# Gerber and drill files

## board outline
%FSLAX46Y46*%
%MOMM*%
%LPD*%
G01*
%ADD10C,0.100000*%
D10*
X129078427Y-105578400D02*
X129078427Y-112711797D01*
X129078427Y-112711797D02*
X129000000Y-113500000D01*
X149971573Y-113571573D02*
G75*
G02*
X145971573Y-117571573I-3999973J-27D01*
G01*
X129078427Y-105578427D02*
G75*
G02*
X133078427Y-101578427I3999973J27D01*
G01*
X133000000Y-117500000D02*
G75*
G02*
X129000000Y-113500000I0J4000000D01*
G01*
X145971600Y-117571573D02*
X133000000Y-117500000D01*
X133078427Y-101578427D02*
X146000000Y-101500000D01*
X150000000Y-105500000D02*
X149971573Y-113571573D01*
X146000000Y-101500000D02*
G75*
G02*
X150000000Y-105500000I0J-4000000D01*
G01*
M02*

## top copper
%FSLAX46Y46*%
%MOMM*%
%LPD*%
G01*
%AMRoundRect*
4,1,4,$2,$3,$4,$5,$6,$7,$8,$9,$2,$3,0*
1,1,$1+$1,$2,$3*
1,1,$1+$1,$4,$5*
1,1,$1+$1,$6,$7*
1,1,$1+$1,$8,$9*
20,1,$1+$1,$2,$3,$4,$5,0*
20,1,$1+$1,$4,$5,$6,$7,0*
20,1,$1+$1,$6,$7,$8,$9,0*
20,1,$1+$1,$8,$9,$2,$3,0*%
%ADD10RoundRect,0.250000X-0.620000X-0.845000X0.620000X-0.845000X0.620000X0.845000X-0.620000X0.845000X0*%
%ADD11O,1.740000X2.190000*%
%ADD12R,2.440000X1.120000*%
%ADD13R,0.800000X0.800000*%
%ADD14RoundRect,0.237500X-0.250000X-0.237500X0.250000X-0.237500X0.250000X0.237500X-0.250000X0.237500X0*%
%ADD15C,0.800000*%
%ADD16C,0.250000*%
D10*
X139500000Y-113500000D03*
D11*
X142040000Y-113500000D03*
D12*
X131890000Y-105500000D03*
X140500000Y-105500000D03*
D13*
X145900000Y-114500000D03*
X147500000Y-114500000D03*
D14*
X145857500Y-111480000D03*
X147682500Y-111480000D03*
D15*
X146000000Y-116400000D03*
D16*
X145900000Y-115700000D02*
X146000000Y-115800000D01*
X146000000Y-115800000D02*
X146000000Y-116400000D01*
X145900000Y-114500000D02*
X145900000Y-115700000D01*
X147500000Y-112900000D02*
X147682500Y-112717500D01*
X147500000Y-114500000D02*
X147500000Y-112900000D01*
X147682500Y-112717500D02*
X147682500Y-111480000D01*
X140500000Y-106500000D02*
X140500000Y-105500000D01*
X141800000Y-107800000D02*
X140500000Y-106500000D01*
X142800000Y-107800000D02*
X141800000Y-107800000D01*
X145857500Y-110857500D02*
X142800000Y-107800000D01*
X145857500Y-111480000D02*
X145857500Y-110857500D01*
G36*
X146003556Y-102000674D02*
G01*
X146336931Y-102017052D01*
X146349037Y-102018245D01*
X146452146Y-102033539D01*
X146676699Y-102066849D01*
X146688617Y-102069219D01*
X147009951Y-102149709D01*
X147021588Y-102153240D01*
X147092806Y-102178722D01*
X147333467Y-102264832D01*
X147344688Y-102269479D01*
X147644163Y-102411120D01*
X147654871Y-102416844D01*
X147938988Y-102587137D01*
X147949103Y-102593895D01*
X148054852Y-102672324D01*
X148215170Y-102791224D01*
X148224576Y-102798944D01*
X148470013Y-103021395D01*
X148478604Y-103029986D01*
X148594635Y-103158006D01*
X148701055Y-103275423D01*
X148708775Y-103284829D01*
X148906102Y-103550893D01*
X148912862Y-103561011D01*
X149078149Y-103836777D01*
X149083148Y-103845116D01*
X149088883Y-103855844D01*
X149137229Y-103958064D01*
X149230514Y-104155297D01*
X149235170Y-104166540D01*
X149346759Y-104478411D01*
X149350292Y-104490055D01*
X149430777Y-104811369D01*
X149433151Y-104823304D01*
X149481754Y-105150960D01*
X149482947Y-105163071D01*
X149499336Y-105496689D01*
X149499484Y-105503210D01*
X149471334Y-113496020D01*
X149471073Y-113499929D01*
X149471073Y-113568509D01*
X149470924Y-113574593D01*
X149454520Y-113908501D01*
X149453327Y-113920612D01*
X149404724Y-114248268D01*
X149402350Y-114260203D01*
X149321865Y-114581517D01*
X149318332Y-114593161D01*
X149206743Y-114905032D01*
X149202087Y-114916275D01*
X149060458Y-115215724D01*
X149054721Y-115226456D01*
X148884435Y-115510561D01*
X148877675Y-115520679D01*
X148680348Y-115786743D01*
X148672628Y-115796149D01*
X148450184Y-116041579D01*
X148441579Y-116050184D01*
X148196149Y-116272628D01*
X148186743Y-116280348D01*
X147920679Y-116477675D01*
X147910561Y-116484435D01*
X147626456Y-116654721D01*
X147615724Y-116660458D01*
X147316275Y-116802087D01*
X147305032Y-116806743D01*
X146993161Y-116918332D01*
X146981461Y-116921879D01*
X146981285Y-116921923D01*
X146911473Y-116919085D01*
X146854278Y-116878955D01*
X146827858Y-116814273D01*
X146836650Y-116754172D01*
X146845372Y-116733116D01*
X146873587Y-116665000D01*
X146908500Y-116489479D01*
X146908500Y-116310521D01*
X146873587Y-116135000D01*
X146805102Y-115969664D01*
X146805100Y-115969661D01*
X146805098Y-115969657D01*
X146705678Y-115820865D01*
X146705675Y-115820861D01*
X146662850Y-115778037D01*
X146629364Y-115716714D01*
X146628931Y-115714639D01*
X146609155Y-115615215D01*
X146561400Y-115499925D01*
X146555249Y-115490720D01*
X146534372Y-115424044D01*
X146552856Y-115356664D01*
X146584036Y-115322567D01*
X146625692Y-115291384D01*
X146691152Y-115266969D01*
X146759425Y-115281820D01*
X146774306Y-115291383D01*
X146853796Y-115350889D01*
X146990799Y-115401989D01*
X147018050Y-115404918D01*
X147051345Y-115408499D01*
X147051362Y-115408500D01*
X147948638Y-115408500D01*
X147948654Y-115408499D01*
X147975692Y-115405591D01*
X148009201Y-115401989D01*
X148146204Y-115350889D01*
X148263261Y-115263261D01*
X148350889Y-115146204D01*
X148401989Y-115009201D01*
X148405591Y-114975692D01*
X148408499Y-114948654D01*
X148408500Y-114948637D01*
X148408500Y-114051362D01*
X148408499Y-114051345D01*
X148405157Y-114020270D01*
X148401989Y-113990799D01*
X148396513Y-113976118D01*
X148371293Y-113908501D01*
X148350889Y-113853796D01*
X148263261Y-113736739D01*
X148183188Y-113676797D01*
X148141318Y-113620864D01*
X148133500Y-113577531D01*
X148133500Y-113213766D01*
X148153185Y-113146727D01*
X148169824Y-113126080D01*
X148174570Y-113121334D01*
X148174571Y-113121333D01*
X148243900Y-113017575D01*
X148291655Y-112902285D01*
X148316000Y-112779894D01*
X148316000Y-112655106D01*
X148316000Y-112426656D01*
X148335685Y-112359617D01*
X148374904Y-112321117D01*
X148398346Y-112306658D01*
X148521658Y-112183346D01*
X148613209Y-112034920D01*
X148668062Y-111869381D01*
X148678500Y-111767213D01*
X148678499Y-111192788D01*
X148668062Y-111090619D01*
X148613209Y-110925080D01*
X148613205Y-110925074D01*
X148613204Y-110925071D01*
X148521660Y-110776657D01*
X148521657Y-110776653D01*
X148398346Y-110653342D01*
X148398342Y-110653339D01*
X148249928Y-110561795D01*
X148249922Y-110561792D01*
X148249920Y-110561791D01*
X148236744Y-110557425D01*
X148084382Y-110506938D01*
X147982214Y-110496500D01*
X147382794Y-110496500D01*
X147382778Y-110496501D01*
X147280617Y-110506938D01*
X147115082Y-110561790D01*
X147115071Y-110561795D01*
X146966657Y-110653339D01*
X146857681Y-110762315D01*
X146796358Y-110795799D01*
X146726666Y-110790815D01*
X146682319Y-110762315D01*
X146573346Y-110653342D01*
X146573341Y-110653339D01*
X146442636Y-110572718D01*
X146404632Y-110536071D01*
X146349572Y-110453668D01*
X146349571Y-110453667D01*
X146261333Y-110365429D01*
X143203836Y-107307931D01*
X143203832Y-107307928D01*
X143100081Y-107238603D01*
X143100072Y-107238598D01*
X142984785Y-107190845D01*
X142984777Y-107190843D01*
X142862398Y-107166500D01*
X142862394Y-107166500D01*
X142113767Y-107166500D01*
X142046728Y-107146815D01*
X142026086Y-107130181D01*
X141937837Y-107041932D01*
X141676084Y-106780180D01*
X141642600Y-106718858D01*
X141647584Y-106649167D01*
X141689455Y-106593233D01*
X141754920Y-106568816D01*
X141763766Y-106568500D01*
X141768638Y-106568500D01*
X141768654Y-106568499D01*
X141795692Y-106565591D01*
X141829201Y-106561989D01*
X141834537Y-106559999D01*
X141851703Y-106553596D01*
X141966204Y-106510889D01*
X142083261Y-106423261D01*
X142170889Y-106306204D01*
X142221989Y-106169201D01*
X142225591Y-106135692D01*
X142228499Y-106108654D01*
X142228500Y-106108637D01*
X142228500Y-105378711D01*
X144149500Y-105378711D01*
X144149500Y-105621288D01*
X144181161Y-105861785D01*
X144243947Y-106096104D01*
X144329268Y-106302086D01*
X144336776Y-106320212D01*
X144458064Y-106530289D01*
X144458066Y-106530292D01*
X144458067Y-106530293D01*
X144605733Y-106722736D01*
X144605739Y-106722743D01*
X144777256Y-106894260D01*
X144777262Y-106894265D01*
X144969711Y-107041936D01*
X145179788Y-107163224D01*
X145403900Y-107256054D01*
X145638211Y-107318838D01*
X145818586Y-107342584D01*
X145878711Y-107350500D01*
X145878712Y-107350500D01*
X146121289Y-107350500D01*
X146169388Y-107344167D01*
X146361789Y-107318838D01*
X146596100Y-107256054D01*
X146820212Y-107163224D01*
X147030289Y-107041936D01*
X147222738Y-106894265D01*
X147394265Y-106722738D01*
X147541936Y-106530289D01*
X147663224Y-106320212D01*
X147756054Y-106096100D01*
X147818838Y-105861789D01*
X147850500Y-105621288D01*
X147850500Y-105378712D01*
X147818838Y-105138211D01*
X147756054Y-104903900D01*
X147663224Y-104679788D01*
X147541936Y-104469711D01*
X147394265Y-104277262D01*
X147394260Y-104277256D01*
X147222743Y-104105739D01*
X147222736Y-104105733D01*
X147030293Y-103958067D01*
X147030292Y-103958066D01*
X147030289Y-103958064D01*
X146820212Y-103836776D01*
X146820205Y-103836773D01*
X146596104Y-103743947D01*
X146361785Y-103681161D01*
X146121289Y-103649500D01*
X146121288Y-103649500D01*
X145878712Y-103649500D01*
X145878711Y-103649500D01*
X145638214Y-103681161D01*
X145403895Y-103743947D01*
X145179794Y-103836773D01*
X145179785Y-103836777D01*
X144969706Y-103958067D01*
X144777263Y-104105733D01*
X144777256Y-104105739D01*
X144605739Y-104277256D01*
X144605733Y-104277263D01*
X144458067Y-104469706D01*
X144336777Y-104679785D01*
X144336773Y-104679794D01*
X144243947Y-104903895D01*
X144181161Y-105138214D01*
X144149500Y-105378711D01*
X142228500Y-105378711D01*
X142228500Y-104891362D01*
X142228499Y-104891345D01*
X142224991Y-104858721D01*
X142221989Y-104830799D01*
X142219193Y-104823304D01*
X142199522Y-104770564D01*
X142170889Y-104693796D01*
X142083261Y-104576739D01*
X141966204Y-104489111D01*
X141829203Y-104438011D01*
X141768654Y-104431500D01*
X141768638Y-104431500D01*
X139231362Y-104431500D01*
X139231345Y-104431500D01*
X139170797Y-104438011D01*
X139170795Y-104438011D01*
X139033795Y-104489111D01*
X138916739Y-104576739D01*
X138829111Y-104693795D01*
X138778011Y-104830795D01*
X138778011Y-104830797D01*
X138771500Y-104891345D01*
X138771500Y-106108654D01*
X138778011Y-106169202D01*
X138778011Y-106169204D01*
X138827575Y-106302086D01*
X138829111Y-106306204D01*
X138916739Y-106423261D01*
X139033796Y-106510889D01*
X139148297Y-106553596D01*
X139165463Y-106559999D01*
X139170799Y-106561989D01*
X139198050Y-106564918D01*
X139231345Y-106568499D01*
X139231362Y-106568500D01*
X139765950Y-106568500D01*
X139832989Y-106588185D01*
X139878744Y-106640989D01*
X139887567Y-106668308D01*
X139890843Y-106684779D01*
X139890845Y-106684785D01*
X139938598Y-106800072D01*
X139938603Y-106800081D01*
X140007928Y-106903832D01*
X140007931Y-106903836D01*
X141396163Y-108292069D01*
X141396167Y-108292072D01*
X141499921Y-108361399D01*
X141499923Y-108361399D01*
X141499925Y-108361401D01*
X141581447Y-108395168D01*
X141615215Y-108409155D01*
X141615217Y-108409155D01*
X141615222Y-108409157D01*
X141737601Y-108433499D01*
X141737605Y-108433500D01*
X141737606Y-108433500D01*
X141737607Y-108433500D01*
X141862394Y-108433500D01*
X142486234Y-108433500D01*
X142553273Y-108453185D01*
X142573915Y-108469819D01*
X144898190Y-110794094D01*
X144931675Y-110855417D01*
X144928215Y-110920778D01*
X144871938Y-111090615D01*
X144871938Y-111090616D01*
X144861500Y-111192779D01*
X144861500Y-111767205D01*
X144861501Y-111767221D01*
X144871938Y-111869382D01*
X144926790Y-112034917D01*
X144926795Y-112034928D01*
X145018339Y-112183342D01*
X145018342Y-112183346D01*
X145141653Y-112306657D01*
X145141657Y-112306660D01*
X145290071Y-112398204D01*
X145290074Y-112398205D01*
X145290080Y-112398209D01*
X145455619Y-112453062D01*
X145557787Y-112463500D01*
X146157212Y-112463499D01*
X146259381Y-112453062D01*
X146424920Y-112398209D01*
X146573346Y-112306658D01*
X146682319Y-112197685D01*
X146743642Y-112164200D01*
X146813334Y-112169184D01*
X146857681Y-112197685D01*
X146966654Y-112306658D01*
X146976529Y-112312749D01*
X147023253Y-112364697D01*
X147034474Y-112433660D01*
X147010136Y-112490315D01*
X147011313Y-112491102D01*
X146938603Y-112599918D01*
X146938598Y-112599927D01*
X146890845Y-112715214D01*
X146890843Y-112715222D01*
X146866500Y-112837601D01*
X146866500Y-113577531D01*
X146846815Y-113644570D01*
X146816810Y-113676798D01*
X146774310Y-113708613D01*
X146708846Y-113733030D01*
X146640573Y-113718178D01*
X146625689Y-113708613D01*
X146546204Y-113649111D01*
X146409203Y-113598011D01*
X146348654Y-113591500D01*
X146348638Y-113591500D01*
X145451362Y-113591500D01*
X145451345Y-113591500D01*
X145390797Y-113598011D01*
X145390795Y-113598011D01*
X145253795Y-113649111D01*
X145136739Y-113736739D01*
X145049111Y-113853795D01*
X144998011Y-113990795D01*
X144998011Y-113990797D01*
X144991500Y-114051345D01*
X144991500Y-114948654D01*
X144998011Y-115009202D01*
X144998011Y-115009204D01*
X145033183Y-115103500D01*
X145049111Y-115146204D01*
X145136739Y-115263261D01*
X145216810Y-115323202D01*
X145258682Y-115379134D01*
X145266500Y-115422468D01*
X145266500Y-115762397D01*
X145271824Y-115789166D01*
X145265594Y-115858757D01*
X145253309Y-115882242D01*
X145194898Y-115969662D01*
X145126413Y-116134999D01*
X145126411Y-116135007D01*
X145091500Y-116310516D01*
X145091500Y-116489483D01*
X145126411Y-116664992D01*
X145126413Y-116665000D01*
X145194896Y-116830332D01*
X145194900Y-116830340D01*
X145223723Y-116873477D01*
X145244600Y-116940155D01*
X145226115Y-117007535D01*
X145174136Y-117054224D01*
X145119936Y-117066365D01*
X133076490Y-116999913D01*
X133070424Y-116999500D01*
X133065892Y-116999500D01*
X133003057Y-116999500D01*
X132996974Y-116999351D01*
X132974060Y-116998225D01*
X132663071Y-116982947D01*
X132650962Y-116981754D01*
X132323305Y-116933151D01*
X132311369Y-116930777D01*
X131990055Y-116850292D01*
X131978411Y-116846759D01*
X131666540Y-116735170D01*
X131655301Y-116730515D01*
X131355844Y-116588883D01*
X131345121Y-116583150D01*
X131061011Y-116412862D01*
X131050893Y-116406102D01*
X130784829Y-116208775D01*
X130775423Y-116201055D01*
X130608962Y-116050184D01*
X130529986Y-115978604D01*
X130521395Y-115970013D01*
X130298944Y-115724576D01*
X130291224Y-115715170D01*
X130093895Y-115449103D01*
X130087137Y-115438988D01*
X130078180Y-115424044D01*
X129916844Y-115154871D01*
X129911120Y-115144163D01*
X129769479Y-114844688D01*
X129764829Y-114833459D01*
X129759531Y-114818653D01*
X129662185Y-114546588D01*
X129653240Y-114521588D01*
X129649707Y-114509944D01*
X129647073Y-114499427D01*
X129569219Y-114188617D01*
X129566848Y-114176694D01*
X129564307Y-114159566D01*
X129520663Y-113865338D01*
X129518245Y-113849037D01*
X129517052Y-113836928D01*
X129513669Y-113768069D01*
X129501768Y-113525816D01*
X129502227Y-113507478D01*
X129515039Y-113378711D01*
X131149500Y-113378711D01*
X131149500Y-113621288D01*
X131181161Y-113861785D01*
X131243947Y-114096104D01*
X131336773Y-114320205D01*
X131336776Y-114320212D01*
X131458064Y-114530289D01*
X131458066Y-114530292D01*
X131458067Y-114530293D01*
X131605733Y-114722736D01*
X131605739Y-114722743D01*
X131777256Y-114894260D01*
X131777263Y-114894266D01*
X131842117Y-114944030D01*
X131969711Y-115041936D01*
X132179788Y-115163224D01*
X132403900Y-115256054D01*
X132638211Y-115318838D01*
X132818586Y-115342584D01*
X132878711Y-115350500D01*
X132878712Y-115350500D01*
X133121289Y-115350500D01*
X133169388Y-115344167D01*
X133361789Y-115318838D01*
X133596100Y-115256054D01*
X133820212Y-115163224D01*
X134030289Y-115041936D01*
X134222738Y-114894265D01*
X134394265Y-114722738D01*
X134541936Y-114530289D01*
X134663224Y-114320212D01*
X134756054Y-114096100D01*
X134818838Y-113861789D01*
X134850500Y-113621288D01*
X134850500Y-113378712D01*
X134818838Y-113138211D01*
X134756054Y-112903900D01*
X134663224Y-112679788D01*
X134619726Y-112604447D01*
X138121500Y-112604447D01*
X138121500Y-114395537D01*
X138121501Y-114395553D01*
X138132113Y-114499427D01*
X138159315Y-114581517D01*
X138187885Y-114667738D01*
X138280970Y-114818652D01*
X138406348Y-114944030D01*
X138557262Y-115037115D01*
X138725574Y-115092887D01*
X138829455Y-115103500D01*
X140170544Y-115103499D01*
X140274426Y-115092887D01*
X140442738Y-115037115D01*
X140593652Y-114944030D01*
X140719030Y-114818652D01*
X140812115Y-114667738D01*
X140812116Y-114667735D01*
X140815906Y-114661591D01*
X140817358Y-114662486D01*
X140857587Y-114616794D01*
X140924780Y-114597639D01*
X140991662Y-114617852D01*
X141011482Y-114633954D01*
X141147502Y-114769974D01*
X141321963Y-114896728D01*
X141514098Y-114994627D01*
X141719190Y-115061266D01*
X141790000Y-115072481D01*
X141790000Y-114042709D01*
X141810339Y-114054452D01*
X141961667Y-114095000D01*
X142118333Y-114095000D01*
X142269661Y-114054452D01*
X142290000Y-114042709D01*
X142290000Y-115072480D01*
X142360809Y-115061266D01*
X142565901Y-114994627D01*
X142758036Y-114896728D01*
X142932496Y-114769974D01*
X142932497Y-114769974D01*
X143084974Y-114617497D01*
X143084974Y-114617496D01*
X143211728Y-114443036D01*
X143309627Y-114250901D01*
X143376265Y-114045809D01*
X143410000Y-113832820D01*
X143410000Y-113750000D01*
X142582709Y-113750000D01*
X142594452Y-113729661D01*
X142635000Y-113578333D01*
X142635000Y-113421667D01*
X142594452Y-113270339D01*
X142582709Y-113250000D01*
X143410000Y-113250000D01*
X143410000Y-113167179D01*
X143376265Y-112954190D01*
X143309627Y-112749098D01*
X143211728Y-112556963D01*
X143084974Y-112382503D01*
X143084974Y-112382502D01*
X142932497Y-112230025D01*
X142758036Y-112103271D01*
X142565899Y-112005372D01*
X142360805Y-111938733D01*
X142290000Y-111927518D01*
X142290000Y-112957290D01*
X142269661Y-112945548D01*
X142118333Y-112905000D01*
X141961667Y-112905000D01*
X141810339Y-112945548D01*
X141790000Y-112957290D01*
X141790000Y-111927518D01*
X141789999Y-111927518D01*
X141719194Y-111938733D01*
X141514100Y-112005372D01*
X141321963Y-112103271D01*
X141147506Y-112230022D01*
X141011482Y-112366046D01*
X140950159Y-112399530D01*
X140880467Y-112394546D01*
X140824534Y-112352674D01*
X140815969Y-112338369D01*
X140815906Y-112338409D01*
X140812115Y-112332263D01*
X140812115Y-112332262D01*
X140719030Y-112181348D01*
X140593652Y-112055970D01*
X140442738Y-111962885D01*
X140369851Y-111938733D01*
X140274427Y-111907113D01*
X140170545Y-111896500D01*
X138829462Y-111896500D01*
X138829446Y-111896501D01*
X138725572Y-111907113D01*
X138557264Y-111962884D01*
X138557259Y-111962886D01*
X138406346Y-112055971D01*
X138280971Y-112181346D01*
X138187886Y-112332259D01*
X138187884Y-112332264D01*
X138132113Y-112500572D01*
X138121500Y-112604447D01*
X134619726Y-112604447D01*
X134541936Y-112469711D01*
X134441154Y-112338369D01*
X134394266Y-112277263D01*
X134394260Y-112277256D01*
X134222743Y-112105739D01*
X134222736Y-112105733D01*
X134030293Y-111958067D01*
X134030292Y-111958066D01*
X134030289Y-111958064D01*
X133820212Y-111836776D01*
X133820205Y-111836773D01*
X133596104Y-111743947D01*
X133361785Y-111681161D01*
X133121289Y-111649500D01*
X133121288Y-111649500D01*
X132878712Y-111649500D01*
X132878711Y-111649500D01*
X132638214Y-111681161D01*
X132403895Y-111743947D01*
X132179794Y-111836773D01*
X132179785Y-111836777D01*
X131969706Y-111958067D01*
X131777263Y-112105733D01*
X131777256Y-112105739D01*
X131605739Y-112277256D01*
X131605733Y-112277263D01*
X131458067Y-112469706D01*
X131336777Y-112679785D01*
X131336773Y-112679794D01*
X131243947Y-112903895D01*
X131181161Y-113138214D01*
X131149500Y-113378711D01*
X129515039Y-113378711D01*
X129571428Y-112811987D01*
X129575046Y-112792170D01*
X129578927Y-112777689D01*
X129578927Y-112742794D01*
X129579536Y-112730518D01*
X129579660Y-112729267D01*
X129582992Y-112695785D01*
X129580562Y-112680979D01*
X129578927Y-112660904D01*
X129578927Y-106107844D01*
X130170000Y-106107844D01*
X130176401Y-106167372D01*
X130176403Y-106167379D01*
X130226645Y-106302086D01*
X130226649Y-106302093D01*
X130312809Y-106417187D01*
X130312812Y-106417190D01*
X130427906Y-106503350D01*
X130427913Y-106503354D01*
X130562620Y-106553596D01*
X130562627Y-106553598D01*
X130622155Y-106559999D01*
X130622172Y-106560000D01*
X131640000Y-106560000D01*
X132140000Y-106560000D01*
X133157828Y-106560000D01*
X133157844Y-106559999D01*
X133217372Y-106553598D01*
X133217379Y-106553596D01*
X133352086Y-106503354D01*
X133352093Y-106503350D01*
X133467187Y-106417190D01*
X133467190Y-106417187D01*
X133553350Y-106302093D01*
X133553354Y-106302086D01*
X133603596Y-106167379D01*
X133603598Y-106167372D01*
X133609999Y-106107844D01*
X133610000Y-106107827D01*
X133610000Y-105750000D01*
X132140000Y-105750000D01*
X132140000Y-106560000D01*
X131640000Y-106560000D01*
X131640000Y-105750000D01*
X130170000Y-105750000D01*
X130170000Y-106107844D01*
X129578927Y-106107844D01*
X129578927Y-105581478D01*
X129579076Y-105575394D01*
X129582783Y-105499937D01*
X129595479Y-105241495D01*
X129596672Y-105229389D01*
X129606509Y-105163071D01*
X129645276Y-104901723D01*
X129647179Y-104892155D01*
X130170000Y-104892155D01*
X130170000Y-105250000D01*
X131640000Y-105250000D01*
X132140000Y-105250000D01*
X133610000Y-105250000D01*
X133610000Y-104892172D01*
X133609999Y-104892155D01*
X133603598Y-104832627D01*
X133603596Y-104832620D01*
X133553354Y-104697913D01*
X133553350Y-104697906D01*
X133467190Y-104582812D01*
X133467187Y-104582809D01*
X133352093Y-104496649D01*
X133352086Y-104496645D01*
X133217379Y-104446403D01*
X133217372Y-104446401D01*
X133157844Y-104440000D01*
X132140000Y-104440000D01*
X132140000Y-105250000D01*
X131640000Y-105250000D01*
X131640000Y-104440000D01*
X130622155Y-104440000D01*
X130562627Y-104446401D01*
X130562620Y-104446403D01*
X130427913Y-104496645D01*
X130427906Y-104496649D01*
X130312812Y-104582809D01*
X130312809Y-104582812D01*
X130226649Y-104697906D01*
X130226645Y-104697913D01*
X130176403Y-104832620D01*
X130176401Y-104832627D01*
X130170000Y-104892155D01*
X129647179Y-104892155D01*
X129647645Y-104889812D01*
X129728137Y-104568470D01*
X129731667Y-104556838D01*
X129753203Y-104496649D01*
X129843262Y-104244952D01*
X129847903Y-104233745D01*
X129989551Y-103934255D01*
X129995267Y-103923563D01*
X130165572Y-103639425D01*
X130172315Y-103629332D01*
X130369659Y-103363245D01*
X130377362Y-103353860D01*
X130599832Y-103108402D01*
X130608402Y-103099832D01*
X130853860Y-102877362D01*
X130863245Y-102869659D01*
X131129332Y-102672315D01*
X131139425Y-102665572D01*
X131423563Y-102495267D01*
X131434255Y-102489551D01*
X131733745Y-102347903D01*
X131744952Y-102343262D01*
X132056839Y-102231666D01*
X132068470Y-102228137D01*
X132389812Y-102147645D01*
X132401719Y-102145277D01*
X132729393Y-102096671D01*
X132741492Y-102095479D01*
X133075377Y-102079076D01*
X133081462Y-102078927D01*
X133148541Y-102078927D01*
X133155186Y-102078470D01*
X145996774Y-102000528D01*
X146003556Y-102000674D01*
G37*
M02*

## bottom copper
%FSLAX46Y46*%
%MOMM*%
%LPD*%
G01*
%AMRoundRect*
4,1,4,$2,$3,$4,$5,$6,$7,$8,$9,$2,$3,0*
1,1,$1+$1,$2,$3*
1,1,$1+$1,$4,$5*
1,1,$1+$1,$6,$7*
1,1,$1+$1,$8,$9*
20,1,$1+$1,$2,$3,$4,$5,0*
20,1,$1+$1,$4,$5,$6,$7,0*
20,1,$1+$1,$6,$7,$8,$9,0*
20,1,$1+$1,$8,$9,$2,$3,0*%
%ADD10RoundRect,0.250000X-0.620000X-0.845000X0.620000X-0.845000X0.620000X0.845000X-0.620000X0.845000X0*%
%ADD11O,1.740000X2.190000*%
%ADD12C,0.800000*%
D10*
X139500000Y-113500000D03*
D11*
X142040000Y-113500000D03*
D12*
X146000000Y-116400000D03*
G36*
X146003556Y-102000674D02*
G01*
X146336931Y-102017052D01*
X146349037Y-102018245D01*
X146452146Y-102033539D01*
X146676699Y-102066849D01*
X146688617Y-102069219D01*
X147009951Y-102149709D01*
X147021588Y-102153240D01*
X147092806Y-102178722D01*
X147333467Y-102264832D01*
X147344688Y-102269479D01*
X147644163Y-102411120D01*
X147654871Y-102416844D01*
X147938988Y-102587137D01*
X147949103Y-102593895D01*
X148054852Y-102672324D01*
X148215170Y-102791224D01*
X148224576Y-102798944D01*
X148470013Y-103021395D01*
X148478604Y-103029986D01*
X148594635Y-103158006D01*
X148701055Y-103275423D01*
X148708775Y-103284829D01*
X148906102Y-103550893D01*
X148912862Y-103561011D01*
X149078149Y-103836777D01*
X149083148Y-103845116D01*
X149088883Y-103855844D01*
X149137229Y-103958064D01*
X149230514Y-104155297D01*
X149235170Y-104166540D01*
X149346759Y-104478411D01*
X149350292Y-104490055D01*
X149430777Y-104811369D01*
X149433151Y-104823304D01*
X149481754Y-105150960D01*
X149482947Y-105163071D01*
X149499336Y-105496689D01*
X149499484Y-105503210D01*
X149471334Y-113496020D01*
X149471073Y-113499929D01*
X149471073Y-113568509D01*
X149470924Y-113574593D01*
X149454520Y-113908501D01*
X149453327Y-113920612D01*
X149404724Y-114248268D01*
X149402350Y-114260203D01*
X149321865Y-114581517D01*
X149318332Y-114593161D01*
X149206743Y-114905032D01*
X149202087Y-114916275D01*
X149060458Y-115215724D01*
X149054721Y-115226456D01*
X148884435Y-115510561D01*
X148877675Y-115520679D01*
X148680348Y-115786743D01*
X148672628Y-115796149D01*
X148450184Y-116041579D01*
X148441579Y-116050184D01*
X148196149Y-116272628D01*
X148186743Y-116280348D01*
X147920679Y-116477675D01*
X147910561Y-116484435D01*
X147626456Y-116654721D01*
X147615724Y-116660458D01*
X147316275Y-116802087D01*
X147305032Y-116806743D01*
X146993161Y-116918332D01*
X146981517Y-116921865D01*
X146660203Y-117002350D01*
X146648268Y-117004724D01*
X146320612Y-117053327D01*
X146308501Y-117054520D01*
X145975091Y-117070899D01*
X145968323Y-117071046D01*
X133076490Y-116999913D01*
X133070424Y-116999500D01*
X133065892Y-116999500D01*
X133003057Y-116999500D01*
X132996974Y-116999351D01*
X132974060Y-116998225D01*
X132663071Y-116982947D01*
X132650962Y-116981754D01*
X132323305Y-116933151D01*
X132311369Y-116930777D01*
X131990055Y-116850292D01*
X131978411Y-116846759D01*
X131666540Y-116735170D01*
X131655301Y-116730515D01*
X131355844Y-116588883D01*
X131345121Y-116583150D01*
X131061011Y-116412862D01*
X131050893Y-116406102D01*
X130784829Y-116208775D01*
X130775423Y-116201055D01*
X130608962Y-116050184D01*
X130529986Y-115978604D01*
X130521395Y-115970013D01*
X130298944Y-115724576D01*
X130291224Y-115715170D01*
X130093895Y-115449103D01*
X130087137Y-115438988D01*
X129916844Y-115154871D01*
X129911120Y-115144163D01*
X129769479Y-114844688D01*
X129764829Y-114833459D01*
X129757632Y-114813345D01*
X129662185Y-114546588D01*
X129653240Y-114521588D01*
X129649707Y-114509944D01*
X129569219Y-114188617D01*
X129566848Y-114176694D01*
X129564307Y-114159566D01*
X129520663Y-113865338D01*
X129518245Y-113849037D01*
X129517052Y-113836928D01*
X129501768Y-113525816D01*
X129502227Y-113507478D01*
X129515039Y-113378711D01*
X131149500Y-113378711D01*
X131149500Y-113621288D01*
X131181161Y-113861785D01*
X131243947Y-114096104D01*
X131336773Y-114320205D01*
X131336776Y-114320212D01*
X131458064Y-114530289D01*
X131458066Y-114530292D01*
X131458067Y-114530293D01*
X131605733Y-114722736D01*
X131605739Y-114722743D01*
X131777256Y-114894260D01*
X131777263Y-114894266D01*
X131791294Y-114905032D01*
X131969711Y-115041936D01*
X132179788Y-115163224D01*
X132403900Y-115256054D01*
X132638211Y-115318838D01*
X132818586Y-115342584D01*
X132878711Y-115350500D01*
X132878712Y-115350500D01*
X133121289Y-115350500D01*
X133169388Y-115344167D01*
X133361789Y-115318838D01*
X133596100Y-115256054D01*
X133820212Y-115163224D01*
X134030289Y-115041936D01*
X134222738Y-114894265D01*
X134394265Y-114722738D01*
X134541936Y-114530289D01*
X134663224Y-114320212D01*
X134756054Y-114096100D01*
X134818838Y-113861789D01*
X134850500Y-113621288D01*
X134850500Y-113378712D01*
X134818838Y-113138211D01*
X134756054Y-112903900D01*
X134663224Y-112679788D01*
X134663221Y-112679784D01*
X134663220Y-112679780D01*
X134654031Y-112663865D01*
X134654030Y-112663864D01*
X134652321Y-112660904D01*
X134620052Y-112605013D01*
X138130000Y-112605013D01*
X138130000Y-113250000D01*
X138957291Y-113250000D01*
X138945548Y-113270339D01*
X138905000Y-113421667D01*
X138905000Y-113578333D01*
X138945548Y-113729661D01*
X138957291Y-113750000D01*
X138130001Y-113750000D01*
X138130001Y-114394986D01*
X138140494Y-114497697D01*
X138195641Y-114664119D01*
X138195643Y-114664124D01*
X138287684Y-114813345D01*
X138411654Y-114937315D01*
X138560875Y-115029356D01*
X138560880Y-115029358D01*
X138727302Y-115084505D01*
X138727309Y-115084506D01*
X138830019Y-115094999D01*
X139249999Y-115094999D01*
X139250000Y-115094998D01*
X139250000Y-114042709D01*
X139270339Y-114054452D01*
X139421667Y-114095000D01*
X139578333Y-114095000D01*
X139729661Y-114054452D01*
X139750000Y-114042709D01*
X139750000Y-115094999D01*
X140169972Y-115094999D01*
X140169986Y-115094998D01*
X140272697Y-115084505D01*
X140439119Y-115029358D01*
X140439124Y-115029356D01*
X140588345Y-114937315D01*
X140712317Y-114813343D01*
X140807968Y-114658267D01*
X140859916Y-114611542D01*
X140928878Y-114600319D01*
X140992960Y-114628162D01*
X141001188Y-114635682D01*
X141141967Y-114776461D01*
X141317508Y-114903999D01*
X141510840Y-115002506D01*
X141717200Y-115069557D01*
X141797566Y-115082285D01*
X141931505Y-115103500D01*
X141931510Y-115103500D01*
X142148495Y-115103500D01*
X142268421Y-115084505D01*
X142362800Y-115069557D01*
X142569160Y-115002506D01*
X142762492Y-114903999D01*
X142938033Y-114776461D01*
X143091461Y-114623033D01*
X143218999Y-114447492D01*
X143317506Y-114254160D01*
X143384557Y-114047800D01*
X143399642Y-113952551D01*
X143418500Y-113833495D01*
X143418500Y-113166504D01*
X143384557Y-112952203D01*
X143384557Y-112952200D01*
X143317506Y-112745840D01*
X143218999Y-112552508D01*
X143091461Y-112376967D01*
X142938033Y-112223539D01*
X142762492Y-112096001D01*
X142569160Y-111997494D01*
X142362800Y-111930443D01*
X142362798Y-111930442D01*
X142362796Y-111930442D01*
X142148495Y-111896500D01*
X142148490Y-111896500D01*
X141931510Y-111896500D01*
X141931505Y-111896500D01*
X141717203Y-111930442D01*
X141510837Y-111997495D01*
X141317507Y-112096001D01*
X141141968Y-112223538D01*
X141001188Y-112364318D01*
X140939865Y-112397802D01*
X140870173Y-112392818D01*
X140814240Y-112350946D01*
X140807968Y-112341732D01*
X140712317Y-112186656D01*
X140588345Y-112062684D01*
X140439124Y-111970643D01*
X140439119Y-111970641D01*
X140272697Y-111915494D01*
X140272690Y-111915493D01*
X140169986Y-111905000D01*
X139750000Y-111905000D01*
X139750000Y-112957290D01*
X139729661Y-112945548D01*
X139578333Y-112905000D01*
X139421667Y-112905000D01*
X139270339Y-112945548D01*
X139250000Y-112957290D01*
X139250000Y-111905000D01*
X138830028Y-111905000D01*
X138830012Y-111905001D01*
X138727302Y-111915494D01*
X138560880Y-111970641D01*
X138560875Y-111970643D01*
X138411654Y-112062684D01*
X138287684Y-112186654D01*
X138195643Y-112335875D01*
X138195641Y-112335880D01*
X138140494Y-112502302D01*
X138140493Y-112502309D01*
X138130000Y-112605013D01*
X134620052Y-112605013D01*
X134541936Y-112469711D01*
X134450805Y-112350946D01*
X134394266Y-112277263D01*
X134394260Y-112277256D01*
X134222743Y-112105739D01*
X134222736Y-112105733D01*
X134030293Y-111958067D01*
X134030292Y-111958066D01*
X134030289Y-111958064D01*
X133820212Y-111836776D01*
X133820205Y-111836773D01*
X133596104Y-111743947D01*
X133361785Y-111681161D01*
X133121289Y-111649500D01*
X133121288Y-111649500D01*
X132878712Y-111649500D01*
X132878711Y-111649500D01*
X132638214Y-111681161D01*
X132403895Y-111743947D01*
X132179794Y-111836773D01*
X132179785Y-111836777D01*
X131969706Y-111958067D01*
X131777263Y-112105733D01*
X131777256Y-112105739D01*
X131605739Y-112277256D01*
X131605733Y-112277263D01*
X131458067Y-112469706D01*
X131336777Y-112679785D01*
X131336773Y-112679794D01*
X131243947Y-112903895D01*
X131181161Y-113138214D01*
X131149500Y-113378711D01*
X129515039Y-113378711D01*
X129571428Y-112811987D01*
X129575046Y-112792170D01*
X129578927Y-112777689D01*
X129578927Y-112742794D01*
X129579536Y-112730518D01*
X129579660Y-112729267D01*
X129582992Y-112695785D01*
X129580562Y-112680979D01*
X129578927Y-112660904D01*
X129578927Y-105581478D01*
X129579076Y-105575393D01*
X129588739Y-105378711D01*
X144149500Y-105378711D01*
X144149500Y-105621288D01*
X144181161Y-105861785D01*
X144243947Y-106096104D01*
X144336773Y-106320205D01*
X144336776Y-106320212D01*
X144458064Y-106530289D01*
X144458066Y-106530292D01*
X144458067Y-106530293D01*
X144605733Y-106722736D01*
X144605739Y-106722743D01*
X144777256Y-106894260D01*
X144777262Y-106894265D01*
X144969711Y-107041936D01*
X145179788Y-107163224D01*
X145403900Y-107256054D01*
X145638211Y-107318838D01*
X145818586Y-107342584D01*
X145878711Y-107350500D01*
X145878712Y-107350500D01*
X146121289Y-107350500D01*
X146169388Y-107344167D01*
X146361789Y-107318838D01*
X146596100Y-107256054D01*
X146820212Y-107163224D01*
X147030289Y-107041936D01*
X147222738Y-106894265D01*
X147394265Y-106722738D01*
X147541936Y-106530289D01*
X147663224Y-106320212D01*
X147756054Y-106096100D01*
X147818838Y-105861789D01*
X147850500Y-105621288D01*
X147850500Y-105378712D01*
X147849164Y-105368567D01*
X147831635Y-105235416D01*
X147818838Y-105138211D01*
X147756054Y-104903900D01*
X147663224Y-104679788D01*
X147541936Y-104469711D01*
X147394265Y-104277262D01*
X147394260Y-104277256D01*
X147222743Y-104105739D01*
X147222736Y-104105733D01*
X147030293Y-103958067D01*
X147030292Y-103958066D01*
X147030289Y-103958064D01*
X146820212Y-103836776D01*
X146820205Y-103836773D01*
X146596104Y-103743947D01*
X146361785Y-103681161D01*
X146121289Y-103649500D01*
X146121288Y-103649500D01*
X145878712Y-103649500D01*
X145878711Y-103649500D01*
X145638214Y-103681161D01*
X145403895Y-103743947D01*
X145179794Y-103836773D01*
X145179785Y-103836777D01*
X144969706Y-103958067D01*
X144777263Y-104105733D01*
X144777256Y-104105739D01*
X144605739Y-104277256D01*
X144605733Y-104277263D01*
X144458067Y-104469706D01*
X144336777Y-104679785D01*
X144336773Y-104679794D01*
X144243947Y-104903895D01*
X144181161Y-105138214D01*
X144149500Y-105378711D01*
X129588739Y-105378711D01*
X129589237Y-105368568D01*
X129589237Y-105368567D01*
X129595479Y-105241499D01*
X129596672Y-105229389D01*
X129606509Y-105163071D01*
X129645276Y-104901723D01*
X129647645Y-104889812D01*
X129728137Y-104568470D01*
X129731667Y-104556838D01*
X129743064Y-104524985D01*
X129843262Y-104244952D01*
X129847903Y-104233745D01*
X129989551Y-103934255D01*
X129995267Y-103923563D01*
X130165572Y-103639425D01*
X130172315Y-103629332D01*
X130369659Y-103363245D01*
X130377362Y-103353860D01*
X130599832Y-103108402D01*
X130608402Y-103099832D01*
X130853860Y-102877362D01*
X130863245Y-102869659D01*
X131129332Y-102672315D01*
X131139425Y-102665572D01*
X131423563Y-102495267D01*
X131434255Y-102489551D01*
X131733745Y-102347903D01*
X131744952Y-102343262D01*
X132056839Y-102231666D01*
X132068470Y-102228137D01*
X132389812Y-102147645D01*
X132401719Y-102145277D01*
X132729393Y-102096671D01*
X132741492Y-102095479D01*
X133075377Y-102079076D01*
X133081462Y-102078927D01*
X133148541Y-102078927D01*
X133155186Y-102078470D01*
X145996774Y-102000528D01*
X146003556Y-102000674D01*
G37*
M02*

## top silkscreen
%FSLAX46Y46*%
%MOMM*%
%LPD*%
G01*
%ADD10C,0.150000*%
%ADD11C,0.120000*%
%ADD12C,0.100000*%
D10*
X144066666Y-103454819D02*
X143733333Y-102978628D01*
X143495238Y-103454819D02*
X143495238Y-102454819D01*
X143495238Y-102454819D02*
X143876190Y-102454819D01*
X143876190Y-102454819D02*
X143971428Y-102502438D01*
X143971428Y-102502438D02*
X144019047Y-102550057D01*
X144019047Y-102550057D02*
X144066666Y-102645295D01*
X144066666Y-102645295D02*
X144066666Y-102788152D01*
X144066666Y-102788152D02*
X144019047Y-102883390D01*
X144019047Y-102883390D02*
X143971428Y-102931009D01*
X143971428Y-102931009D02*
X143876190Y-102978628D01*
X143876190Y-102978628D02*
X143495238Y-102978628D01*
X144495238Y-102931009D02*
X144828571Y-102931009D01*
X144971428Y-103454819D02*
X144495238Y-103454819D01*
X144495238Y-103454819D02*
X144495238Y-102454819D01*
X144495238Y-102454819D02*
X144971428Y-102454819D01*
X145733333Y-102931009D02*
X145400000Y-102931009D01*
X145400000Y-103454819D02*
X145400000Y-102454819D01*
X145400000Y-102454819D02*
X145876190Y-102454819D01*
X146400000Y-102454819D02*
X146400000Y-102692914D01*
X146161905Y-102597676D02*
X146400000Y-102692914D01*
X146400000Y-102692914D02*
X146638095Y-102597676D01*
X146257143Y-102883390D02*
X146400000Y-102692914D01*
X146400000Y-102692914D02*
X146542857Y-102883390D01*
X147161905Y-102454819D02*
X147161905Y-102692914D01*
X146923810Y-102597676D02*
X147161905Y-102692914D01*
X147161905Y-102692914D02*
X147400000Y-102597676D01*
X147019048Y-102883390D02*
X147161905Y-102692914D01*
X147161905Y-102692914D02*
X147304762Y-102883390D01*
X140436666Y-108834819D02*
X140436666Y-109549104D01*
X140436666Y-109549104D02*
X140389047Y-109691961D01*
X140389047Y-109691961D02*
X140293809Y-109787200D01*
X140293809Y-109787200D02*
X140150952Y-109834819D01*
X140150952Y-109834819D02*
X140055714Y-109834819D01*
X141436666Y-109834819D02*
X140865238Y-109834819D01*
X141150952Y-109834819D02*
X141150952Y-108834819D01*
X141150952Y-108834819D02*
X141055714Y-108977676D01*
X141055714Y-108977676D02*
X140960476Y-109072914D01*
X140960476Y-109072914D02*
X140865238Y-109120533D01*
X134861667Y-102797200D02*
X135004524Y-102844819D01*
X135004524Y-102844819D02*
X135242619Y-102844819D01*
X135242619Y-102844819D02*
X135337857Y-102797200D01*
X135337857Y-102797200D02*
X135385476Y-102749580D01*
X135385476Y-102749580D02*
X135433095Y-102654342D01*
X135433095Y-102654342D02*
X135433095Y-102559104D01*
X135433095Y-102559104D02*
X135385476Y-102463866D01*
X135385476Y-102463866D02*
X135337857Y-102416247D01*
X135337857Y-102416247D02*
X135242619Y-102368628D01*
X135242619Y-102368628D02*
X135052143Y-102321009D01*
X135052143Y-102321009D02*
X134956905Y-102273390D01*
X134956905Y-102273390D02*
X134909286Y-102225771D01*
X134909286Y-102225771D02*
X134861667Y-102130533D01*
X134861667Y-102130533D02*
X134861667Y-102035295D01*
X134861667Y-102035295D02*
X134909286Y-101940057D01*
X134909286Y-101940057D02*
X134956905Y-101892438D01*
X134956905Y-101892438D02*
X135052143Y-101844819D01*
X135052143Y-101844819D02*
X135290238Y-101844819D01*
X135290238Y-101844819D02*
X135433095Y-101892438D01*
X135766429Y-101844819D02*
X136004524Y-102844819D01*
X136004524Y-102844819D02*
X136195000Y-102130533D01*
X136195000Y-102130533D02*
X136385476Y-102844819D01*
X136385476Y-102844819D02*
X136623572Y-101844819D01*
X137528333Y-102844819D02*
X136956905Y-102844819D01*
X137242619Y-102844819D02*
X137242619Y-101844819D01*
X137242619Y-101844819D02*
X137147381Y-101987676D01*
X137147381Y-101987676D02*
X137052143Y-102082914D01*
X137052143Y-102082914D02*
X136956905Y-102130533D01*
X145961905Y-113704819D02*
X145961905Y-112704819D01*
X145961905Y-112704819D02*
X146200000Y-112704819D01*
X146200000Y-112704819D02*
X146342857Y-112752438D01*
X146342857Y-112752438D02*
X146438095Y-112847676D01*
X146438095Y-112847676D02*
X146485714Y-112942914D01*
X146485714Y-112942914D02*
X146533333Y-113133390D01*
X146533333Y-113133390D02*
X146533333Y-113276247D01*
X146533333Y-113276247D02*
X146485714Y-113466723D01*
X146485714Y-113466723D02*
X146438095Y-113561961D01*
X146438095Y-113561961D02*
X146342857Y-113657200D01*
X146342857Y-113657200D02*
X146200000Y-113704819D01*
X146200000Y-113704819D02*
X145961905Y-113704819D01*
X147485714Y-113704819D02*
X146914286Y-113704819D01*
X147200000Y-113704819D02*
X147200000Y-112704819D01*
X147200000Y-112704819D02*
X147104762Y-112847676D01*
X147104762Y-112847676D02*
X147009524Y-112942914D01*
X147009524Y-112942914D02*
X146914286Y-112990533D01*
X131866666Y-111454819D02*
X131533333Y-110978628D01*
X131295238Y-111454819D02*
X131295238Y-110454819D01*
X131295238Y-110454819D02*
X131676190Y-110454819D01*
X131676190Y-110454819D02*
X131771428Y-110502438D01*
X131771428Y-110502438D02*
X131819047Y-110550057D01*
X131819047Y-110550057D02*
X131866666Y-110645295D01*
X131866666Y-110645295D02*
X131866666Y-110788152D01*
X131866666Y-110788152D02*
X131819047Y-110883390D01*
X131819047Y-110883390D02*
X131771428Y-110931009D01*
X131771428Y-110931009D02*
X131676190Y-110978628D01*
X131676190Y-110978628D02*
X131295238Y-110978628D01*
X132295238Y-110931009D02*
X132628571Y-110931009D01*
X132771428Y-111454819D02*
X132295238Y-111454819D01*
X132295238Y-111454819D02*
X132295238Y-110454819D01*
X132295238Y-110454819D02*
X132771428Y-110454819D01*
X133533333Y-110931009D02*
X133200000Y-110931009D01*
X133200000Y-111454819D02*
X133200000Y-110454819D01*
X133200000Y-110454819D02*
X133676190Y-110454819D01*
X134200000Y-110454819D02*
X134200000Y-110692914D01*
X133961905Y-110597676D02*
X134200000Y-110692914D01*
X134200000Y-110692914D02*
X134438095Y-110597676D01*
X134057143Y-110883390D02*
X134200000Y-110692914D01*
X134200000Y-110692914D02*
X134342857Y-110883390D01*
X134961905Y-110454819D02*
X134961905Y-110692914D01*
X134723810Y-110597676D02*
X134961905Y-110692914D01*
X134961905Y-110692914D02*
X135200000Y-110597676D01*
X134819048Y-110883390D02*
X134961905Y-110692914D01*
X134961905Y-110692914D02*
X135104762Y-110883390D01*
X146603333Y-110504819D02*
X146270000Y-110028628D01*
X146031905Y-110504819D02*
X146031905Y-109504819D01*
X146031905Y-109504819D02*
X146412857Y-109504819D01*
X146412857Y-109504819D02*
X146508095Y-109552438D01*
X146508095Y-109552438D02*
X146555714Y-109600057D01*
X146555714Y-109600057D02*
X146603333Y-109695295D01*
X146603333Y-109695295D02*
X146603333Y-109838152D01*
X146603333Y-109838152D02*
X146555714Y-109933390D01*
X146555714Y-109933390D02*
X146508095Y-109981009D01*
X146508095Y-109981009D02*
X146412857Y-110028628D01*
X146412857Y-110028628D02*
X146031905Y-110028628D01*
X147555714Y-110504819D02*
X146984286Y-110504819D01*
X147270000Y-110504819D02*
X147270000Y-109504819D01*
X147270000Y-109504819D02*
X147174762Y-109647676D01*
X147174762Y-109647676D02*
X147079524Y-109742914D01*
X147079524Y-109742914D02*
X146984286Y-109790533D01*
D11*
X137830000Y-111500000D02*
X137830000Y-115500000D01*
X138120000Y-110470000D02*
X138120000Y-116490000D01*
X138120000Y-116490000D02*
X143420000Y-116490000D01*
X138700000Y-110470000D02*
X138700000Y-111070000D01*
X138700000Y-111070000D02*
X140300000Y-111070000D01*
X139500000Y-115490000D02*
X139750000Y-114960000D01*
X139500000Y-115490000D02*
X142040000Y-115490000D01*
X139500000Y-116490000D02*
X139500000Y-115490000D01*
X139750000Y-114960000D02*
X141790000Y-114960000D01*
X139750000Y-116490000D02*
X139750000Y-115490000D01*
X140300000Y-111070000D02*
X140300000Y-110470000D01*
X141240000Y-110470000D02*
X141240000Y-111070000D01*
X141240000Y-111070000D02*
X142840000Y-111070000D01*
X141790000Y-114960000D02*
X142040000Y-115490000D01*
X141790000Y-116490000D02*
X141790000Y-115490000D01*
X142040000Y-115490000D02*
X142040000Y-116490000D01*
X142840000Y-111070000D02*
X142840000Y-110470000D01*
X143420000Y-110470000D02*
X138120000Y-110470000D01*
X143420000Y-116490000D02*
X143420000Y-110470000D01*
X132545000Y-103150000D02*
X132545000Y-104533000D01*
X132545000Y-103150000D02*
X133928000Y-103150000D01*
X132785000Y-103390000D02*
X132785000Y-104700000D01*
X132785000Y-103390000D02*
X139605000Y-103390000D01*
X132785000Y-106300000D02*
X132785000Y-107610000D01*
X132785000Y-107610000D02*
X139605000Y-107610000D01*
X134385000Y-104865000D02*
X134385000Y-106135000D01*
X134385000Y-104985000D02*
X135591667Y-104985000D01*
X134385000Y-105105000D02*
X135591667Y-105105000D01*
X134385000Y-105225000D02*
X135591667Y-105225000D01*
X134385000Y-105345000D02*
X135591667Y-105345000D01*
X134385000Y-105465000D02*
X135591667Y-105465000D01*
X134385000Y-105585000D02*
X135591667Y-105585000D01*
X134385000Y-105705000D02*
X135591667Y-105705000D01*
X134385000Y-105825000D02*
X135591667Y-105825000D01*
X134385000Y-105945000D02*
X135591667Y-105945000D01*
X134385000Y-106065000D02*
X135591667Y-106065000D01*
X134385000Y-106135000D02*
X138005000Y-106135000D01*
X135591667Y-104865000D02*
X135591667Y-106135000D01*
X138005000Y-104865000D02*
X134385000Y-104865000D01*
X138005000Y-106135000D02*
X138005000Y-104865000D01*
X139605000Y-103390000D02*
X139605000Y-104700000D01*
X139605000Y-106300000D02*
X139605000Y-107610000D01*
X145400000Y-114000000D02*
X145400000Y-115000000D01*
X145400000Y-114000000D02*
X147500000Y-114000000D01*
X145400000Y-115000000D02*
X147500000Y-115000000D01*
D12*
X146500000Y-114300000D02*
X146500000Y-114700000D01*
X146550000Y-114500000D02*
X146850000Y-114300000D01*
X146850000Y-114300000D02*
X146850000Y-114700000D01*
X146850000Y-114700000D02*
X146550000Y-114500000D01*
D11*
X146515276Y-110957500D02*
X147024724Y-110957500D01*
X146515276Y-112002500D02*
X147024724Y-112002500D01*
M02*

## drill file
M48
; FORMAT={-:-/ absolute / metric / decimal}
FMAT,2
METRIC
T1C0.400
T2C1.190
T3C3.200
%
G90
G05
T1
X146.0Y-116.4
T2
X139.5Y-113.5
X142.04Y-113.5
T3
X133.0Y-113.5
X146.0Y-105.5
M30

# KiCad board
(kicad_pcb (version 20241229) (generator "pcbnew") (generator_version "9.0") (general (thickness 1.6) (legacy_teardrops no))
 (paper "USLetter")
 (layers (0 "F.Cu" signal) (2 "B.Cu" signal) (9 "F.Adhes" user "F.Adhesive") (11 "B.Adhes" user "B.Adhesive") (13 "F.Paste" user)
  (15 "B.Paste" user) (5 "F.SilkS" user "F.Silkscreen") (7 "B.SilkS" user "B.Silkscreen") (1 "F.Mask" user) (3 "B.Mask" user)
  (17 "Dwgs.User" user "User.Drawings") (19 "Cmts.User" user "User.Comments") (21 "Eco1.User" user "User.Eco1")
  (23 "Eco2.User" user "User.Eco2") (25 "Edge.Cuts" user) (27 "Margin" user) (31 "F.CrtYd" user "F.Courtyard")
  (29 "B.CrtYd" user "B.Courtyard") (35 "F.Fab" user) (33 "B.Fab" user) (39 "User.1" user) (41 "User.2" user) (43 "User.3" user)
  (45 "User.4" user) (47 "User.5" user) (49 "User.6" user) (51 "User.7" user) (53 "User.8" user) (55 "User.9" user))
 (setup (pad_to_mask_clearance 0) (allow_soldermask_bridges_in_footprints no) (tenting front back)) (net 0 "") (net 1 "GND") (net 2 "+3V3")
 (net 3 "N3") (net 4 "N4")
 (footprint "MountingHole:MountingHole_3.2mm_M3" (layer "F.Cu") (at 146 105.5)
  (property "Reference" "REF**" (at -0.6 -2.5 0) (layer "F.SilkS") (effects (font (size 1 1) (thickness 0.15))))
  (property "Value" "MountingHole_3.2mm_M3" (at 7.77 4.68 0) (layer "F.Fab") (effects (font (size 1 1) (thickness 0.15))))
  (pad "" np_thru_hole circle (at 0 0) (size 3.2 3.2) (drill 3.2) (layers "*.Cu" "*.Mask")))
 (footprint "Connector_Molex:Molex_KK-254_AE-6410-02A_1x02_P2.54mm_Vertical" (layer "F.Cu") (at 139.5 113.5)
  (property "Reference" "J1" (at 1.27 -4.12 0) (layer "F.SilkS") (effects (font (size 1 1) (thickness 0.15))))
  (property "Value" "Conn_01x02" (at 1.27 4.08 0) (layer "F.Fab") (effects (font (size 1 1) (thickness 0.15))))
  (fp_line (start -1.67 -2) (end -1.67 2) (stroke (width 0.12) (type solid)) (layer "F.SilkS"))
  (fp_line (start -1.38 -3.03) (end -1.38 2.99) (stroke (width 0.12) (type solid)) (layer "F.SilkS"))
  (fp_line (start -1.38 2.99) (end 3.92 2.99) (stroke (width 0.12) (type solid)) (layer "F.SilkS"))
  (fp_line (start -0.8 -3.03) (end -0.8 -2.43) (stroke (width 0.12) (type solid)) (layer "F.SilkS"))
  (fp_line (start -0.8 -2.43) (end 0.8 -2.43) (stroke (width 0.12) (type solid)) (layer "F.SilkS"))
  (fp_line (start 0 1.99) (end 0.25 1.46) (stroke (width 0.12) (type solid)) (layer "F.SilkS"))
  (fp_line (start 0 1.99) (end 2.54 1.99) (stroke (width 0.12) (type solid)) (layer "F.SilkS"))
  (fp_line (start 0 2.99) (end 0 1.99) (stroke (width 0.12) (type solid)) (layer "F.SilkS"))
  (fp_line (start 0.25 1.46) (end 2.29 1.46) (stroke (width 0.12) (type solid)) (layer "F.SilkS"))
  (fp_line (start 0.25 2.99) (end 0.25 1.99) (stroke (width 0.12) (type solid)) (layer "F.SilkS"))
  (fp_line (start 0.8 -2.43) (end 0.8 -3.03) (stroke (width 0.12) (type solid)) (layer "F.SilkS"))
  (fp_line (start 1.74 -3.03) (end 1.74 -2.43) (stroke (width 0.12) (type solid)) (layer "F.SilkS"))
  (fp_line (start 1.74 -2.43) (end 3.34 -2.43) (stroke (width 0.12) (type solid)) (layer "F.SilkS"))
  (fp_line (start 2.29 1.46) (end 2.54 1.99) (stroke (width 0.12) (type solid)) (layer "F.SilkS"))
  (fp_line (start 2.29 2.99) (end 2.29 1.99) (stroke (width 0.12) (type solid)) (layer "F.SilkS"))
  (fp_line (start 2.54 1.99) (end 2.54 2.99) (stroke (width 0.12) (type solid)) (layer "F.SilkS"))
  (fp_line (start 3.34 -2.43) (end 3.34 -3.03) (stroke (width 0.12) (type solid)) (layer "F.SilkS"))
  (fp_line (start 3.92 -3.03) (end -1.38 -3.03) (stroke (width 0.12) (type solid)) (layer "F.SilkS"))
  (fp_line (start 3.92 2.99) (end 3.92 -3.03) (stroke (width 0.12) (type solid)) (layer "F.SilkS"))
  (pad "1" thru_hole roundrect (at 0 0) (size 1.74 2.19) (drill 1.19) (layers "*.Cu" "*.Mask") (remove_unused_layers no)
   (roundrect_rratio 0.143678) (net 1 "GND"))
  (pad "2" thru_hole oval (at 2.54 0) (size 1.74 2.19) (drill 1.19) (layers "*.Cu" "*.Mask") (remove_unused_layers no) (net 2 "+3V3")))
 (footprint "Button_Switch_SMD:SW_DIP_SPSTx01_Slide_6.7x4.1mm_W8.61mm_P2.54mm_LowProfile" (layer "F.Cu") (at 136.195 105.5)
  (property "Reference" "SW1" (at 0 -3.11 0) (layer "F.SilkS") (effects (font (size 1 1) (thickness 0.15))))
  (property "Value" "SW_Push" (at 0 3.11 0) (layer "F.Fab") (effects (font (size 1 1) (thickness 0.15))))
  (fp_line (start -3.65 -2.35) (end -3.65 -0.967) (stroke (width 0.12) (type solid)) (layer "F.SilkS"))
  (fp_line (start -3.65 -2.35) (end -2.267 -2.35) (stroke (width 0.12) (type solid)) (layer "F.SilkS"))
  (fp_line (start -3.41 -2.11) (end -3.41 -0.8) (stroke (width 0.12) (type solid)) (layer "F.SilkS"))
  (fp_line (start -3.41 -2.11) (end 3.41 -2.11) (stroke (width 0.12) (type solid)) (layer "F.SilkS"))
  (fp_line (start -3.41 0.8) (end -3.41 2.11) (stroke (width 0.12) (type solid)) (layer "F.SilkS"))
  (fp_line (start -3.41 2.11) (end 3.41 2.11) (stroke (width 0.12) (type solid)) (layer "F.SilkS"))
  (fp_line (start -1.81 -0.635) (end -1.81 0.635) (stroke (width 0.12) (type solid)) (layer "F.SilkS"))
  (fp_line (start -1.81 -0.515) (end -0.603333 -0.515) (stroke (width 0.12) (type solid)) (layer "F.SilkS"))
  (fp_line (start -1.81 -0.395) (end -0.603333 -0.395) (stroke (width 0.12) (type solid)) (layer "F.SilkS"))
  (fp_line (start -1.81 -0.275) (end -0.603333 -0.275) (stroke (width 0.12) (type solid)) (layer "F.SilkS"))
  (fp_line (start -1.81 -0.155) (end -0.603333 -0.155) (stroke (width 0.12) (type solid)) (layer "F.SilkS"))
  (fp_line (start -1.81 -0.035) (end -0.603333 -0.035) (stroke (width 0.12) (type solid)) (layer "F.SilkS"))
  (fp_line (start -1.81 0.085) (end -0.603333 0.085) (stroke (width 0.12) (type solid)) (layer "F.SilkS"))
  (fp_line (start -1.81 0.205) (end -0.603333 0.205) (stroke (width 0.12) (type solid)) (layer "F.SilkS"))
  (fp_line (start -1.81 0.325) (end -0.603333 0.325) (stroke (width 0.12) (type solid)) (layer "F.SilkS"))
  (fp_line (start -1.81 0.445) (end -0.603333 0.445) (stroke (width 0.12) (type solid)) (layer "F.SilkS"))
  (fp_line (start -1.81 0.565) (end -0.603333 0.565) (stroke (width 0.12) (type solid)) (layer "F.SilkS"))
  (fp_line (start -1.81 0.635) (end 1.81 0.635) (stroke (width 0.12) (type solid)) (layer "F.SilkS"))
  (fp_line (start -0.603333 -0.635) (end -0.603333 0.635) (stroke (width 0.12) (type solid)) (layer "F.SilkS"))
  (fp_line (start 1.81 -0.635) (end -1.81 -0.635) (stroke (width 0.12) (type solid)) (layer "F.SilkS"))
  (fp_line (start 1.81 0.635) (end 1.81 -0.635) (stroke (width 0.12) (type solid)) (layer "F.SilkS"))
  (fp_line (start 3.41 -2.11) (end 3.41 -0.8) (stroke (width 0.12) (type solid)) (layer "F.SilkS"))
  (fp_line (start 3.41 0.8) (end 3.41 2.11) (stroke (width 0.12) (type solid)) (layer "F.SilkS"))
  (pad "1" smd rect (at -4.305 0) (size 2.44 1.12) (layers "F.Cu" "F.Mask" "F.Paste") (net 2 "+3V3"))
  (pad "2" smd rect (at 4.305 0) (size 2.44 1.12) (layers "F.Cu" "F.Mask" "F.Paste") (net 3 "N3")))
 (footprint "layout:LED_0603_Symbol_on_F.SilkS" (layer "F.Cu") (at 146.7 114.5)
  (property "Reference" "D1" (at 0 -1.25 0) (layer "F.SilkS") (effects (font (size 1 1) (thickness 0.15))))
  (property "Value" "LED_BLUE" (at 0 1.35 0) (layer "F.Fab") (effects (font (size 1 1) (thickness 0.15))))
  (fp_line (start -1.3 -0.5) (end -1.3 0.5) (stroke (width 0.12) (type solid)) (layer "F.SilkS"))
  (fp_line (start -1.3 -0.5) (end 0.8 -0.5) (stroke (width 0.12) (type solid)) (layer "F.SilkS"))
  (fp_line (start -1.3 0.5) (end 0.8 0.5) (stroke (width 0.12) (type solid)) (layer "F.SilkS"))
  (fp_line (start -0.2 -0.2) (end -0.2 0.2) (stroke (width 0.1) (type solid)) (layer "F.SilkS"))
  (fp_line (start -0.15 0) (end 0.15 -0.2) (stroke (width 0.1) (type solid)) (layer "F.SilkS"))
  (fp_line (start 0.15 -0.2) (end 0.15 0.2) (stroke (width 0.1) (type solid)) (layer "F.SilkS"))
  (fp_line (start 0.15 0.2) (end -0.15 0) (stroke (width 0.1) (type solid)) (layer "F.SilkS"))
  (pad "1" smd rect (at -0.8 0 180) (size 0.8 0.8) (layers "F.Cu" "F.Mask" "F.Paste") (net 1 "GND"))
  (pad "2" smd rect (at 0.8 0 180) (size 0.8 0.8) (layers "F.Cu" "F.Mask" "F.Paste") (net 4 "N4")))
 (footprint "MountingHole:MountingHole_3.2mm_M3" (layer "F.Cu") (at 133 113.5)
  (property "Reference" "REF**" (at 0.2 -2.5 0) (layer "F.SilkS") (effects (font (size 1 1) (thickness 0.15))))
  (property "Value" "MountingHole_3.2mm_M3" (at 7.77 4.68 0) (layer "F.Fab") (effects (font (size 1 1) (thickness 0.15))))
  (pad "" np_thru_hole circle (at 0 0) (size 3.2 3.2) (drill 3.2) (layers "*.Cu" "*.Mask")))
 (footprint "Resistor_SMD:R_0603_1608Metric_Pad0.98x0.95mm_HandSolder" (layer "F.Cu") (at 146.77 111.48)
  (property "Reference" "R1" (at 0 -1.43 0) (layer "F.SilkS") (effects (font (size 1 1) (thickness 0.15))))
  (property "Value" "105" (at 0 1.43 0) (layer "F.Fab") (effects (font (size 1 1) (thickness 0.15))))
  (fp_line (start -0.254724 -0.5225) (end 0.254724 -0.5225) (stroke (width 0.12) (type solid)) (layer "F.SilkS"))
  (fp_line (start -0.254724 0.5225) (end 0.254724 0.5225) (stroke (width 0.12) (type solid)) (layer "F.SilkS"))
  (pad "1" smd roundrect (at -0.9125 0) (size 0.975 0.95) (layers "F.Cu" "F.Mask" "F.Paste") (roundrect_rratio 0.25) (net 3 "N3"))
  (pad "2" smd roundrect (at 0.9125 0) (size 0.975 0.95) (layers "F.Cu" "F.Mask" "F.Paste") (roundrect_rratio 0.25) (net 4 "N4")))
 (gr_line (start 129.078427 105.5784) (end 129.078427 112.711797) (stroke (width 0.1) (type default)) (layer "Edge.Cuts"))
 (gr_line (start 129.078427 112.711797) (end 129 113.5) (stroke (width 0.1) (type default)) (layer "Edge.Cuts"))
 (gr_arc (start 149.971573 113.571573) (mid 148.8 116.4) (end 145.971573 117.571573) (stroke (width 0.1) (type default)) (layer "Edge.Cuts"))
 (gr_arc (start 129.078427 105.578427) (mid 130.25 102.75) (end 133.078427 101.578427) (stroke (width 0.1) (type default))
  (layer "Edge.Cuts"))
 (gr_arc (start 133 117.5) (mid 130.171573 116.328427) (end 129 113.5) (stroke (width 0.1) (type default)) (layer "Edge.Cuts"))
 (gr_line (start 145.9716 117.571573) (end 133 117.5) (stroke (width 0.1) (type default)) (layer "Edge.Cuts"))
 (gr_line (start 133.078427 101.578427) (end 146 101.5) (stroke (width 0.1) (type default)) (layer "Edge.Cuts"))
 (gr_line (start 150 105.5) (end 149.971573 113.571573) (stroke (width 0.1) (type default)) (layer "Edge.Cuts"))
 (gr_arc (start 146 101.5) (mid 148.828427 102.671573) (end 150 105.5) (stroke (width 0.1) (type default)) (layer "Edge.Cuts"))
 (segment (start 145.9 115.7) (end 146 115.8) (width 0.25) (layer "F.Cu") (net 1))
 (segment (start 146 115.8) (end 146 116.4) (width 0.25) (layer "F.Cu") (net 1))
 (segment (start 145.9 114.5) (end 145.9 115.7) (width 0.25) (layer "F.Cu") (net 1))
 (via (at 146 116.4) (size 0.8) (drill 0.4) (layers "F.Cu" "B.Cu") (free yes) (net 1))
 (segment (start 147.5 112.9) (end 147.6825 112.7175) (width 0.25) (layer "F.Cu") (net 4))
 (segment (start 147.5 114.5) (end 147.5 112.9) (width 0.25) (layer "F.Cu") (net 4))
 (segment (start 147.6825 112.7175) (end 147.6825 111.48) (width 0.25) (layer "F.Cu") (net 4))
 (segment (start 140.5 106.5) (end 140.5 105.5) (width 0.25) (layer "F.Cu") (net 3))
 (segment (start 141.8 107.8) (end 140.5 106.5) (width 0.25) (layer "F.Cu") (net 3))
 (segment (start 142.8 107.8) (end 141.8 107.8) (width 0.25) (layer "F.Cu") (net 3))
 (segment (start 145.8575 110.8575) (end 142.8 107.8) (width 0.25) (layer "F.Cu") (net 3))
 (segment (start 145.8575 111.48) (end 145.8575 110.8575) (width 0.25) (layer "F.Cu") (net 3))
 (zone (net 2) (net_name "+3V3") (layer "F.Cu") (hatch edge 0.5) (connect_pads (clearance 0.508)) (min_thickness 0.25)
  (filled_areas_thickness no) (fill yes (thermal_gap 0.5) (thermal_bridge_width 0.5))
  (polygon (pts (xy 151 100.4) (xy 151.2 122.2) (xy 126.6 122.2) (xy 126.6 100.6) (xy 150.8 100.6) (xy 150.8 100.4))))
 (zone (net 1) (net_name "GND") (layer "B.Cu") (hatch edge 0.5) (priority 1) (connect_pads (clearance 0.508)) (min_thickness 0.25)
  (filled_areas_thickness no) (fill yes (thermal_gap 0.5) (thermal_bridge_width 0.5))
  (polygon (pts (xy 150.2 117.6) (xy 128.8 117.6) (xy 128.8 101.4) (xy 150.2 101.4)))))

